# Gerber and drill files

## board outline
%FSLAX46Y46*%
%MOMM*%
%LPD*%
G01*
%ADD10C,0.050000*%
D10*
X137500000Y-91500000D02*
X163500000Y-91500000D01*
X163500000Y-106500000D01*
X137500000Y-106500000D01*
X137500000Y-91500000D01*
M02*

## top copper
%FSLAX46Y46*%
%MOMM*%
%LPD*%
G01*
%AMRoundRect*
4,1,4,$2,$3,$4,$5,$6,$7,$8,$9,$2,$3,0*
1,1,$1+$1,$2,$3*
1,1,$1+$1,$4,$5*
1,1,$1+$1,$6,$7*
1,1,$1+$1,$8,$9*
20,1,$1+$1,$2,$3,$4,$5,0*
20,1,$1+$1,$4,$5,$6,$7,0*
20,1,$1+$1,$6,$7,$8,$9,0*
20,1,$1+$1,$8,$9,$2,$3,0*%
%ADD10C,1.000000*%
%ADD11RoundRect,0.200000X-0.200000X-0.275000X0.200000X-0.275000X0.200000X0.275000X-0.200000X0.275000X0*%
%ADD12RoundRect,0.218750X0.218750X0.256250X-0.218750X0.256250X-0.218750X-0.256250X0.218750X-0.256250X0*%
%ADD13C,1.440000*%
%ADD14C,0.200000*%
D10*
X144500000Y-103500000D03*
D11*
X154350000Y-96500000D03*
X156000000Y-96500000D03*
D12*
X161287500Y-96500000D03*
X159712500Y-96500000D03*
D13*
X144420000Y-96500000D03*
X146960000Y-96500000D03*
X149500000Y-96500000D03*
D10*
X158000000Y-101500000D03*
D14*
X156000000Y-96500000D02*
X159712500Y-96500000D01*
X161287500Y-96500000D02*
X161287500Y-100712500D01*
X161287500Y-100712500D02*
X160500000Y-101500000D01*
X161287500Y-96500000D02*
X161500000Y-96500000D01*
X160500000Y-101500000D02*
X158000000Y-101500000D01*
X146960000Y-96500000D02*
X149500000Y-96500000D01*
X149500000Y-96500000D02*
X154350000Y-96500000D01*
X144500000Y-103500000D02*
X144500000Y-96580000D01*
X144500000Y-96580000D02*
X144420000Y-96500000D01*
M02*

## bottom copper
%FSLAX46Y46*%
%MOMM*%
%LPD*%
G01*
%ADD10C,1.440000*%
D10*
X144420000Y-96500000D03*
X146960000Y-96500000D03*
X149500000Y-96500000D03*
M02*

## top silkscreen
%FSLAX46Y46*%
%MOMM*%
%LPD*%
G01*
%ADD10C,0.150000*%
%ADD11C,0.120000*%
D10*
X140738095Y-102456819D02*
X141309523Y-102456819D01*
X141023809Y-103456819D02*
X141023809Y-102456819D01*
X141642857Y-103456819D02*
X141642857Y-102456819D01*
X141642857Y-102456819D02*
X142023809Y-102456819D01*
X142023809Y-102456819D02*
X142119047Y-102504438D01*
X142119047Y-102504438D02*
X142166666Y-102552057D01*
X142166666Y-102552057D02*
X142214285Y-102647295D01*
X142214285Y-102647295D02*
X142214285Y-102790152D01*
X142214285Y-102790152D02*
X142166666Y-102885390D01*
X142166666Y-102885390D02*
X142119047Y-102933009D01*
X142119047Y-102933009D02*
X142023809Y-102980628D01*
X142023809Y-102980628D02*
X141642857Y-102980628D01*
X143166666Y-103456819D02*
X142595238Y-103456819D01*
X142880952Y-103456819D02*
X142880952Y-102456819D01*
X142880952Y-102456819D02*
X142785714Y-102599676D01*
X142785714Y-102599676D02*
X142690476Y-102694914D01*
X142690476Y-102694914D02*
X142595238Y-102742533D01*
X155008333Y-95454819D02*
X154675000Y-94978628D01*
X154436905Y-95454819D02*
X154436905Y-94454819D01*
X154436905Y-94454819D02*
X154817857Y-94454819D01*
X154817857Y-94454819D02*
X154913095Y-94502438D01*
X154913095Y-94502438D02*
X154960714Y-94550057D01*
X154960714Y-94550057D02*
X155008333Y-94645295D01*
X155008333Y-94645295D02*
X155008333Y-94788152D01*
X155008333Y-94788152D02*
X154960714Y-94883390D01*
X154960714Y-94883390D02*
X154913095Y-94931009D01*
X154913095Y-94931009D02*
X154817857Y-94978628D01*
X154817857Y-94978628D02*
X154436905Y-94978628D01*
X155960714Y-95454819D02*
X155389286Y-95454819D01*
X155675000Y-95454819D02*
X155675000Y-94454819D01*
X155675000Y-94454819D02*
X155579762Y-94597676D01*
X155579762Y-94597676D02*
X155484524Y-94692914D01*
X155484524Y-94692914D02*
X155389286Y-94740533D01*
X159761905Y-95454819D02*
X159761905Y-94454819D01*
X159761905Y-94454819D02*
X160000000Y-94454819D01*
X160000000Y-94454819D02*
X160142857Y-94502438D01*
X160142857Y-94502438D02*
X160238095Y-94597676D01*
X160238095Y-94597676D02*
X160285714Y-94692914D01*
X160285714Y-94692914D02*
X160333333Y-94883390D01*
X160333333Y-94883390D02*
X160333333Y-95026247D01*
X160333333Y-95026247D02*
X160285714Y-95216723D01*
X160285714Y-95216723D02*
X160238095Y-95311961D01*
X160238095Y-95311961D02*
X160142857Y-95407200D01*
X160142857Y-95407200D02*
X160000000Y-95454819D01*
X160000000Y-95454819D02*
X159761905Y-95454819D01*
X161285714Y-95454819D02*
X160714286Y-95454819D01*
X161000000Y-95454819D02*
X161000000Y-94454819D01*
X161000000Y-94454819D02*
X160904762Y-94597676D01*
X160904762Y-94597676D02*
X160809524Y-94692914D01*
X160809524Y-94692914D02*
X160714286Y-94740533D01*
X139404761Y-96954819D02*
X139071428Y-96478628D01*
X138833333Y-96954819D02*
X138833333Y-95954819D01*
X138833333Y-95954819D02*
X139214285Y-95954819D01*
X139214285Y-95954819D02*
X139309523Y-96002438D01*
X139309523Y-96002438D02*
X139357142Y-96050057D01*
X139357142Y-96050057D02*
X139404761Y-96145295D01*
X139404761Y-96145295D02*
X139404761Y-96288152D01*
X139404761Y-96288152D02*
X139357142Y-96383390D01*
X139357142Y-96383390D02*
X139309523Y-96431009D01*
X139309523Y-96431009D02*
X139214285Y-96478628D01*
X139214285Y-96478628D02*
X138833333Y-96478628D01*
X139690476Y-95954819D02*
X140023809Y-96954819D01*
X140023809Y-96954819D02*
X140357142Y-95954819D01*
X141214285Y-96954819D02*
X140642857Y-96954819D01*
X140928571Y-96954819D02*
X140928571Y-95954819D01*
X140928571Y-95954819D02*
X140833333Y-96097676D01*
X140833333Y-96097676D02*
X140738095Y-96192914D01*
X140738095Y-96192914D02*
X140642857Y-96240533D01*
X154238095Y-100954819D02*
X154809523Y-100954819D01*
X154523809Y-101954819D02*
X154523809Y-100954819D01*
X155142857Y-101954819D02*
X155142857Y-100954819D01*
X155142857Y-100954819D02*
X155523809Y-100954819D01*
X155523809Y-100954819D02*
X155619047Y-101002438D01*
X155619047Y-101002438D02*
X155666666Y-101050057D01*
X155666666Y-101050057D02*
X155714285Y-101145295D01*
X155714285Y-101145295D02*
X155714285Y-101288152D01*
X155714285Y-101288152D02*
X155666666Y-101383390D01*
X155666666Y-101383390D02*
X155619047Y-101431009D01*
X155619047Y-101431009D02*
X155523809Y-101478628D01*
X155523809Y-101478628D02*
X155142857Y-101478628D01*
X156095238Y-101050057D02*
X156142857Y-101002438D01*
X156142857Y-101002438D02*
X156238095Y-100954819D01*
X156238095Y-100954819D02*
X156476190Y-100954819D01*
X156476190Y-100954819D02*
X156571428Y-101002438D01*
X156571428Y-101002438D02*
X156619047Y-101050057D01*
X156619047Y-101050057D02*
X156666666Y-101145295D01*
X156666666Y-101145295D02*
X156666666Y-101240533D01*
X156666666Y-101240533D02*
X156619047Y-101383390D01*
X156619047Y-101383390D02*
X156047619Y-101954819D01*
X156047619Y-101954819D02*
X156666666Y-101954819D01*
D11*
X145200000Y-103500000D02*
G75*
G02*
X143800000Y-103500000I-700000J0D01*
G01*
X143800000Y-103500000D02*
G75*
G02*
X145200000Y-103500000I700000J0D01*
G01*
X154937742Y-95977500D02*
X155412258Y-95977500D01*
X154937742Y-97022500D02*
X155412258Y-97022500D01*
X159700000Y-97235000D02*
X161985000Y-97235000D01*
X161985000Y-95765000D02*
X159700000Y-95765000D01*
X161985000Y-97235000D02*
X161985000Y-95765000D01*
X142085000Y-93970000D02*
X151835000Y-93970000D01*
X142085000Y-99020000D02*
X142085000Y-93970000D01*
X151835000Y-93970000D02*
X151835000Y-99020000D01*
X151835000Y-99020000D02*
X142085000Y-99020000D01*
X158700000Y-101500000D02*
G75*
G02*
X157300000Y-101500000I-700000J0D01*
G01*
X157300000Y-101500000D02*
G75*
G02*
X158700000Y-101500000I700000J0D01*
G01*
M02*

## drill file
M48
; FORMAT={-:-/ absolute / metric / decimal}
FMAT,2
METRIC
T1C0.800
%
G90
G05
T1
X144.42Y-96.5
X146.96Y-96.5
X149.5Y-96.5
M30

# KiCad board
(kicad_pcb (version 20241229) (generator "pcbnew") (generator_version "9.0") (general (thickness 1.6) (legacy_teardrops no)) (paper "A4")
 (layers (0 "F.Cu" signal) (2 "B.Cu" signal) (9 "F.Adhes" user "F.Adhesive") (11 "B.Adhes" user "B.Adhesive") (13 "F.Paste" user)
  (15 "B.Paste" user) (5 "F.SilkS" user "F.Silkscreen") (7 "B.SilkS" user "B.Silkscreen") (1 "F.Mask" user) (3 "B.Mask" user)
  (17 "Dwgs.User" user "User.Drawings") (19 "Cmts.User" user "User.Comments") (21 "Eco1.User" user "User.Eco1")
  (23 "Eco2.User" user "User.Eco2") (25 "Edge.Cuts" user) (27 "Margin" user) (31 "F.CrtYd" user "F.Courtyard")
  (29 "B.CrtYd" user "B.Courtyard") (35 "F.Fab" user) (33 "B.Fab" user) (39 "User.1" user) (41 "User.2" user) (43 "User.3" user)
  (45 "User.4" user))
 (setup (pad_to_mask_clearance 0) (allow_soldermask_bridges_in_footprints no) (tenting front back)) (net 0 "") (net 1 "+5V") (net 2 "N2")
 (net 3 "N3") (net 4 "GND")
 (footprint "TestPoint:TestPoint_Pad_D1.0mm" (layer "F.Cu") (at 144.5 103.5)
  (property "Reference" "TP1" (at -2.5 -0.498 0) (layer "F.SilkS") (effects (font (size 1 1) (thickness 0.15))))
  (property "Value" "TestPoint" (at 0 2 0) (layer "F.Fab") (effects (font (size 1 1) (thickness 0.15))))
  (fp_circle (center 0 0) (end 0 0.7) (stroke (width 0.12) (type solid)) (fill no) (layer "F.SilkS"))
  (pad "1" smd circle (at 0 0) (size 1 1) (layers "F.Cu" "F.Mask") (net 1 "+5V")))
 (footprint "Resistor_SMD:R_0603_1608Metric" (layer "F.Cu") (at 155.175 96.5)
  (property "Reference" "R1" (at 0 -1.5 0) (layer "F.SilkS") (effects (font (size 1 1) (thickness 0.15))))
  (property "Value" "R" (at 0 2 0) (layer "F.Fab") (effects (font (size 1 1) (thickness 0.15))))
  (fp_line (start -0.237258 -0.5225) (end 0.237258 -0.5225) (stroke (width 0.12) (type solid)) (layer "F.SilkS"))
  (fp_line (start -0.237258 0.5225) (end 0.237258 0.5225) (stroke (width 0.12) (type solid)) (layer "F.SilkS"))
  (pad "1" smd roundrect (at -0.825 0) (size 0.8 0.95) (layers "F.Cu" "F.Mask" "F.Paste") (roundrect_rratio 0.25) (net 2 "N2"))
  (pad "2" smd roundrect (at 0.825 0) (size 0.8 0.95) (layers "F.Cu" "F.Mask" "F.Paste") (roundrect_rratio 0.25) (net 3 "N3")))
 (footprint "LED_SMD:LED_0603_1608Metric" (layer "F.Cu") (at 160.5 96.5 180)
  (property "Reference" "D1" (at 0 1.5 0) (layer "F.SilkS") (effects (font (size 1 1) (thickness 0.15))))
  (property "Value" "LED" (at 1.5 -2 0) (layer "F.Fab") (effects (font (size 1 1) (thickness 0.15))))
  (fp_line (start 0.8 -0.735) (end -1.485 -0.735) (stroke (width 0.12) (type solid)) (layer "F.SilkS"))
  (fp_line (start -1.485 0.735) (end 0.8 0.735) (stroke (width 0.12) (type solid)) (layer "F.SilkS"))
  (fp_line (start -1.485 -0.735) (end -1.485 0.735) (stroke (width 0.12) (type solid)) (layer "F.SilkS"))
  (pad "1" smd roundrect (at -0.7875 0 180) (size 0.875 0.95) (layers "F.Cu" "F.Mask" "F.Paste") (roundrect_rratio 0.25) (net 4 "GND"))
  (pad "2" smd roundrect (at 0.7875 0 180) (size 0.875 0.95) (layers "F.Cu" "F.Mask" "F.Paste") (roundrect_rratio 0.25) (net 3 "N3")))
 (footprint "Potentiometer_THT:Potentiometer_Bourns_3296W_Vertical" (layer "F.Cu") (at 144.42 96.5 180)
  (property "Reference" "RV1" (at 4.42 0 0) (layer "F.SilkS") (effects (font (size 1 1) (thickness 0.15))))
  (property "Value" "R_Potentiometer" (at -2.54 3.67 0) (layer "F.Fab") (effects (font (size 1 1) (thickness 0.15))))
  (fp_line (start 2.335 2.53) (end -7.415 2.53) (stroke (width 0.12) (type solid)) (layer "F.SilkS"))
  (fp_line (start 2.335 -2.52) (end 2.335 2.53) (stroke (width 0.12) (type solid)) (layer "F.SilkS"))
  (fp_line (start -7.415 2.53) (end -7.415 -2.52) (stroke (width 0.12) (type solid)) (layer "F.SilkS"))
  (fp_line (start -7.415 -2.52) (end 2.335 -2.52) (stroke (width 0.12) (type solid)) (layer "F.SilkS"))
  (pad "1" thru_hole circle (at 0 0 180) (size 1.44 1.44) (drill 0.8) (layers "*.Cu" "*.Mask") (remove_unused_layers no) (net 1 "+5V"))
  (pad "2" thru_hole circle (at -2.54 0 180) (size 1.44 1.44) (drill 0.8) (layers "*.Cu" "*.Mask") (remove_unused_layers no) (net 2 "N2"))
  (pad "3" thru_hole circle (at -5.08 0 180) (size 1.44 1.44) (drill 0.8) (layers "*.Cu" "*.Mask") (remove_unused_layers no) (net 2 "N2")))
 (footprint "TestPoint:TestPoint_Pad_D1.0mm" (layer "F.Cu") (at 158 101.5)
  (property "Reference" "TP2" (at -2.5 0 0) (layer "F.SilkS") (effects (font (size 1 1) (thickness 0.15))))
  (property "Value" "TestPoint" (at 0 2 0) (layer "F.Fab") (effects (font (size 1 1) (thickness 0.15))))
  (fp_circle (center 0 0) (end 0 0.7) (stroke (width 0.12) (type solid)) (fill no) (layer "F.SilkS"))
  (pad "1" smd circle (at 0 0) (size 1 1) (layers "F.Cu" "F.Mask") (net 4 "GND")))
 (gr_rect (start 137.5 91.5) (end 163.5 106.5) (stroke (width 0.05) (type default)) (fill no) (layer "Edge.Cuts"))
 (segment (start 156 96.5) (end 159.7125 96.5) (width 0.2) (layer "F.Cu") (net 3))
 (segment (start 161.2875 96.5) (end 161.2875 100.7125) (width 0.2) (layer "F.Cu") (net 4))
 (segment (start 161.2875 100.7125) (end 160.5 101.5) (width 0.2) (layer "F.Cu") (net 4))
 (segment (start 161.2875 96.5) (end 161.5 96.5) (width 0.2) (layer "F.Cu") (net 4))
 (segment (start 160.5 101.5) (end 158 101.5) (width 0.2) (layer "F.Cu") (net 4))
 (segment (start 146.96 96.5) (end 149.5 96.5) (width 0.2) (layer "F.Cu") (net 2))
 (segment (start 149.5 96.5) (end 154.35 96.5) (width 0.2) (layer "F.Cu") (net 2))
 (segment (start 144.5 103.5) (end 144.5 96.58) (width 0.2) (layer "F.Cu") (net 1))
 (segment (start 144.5 96.58) (end 144.42 96.5) (width 0.2) (layer "F.Cu") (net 1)))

